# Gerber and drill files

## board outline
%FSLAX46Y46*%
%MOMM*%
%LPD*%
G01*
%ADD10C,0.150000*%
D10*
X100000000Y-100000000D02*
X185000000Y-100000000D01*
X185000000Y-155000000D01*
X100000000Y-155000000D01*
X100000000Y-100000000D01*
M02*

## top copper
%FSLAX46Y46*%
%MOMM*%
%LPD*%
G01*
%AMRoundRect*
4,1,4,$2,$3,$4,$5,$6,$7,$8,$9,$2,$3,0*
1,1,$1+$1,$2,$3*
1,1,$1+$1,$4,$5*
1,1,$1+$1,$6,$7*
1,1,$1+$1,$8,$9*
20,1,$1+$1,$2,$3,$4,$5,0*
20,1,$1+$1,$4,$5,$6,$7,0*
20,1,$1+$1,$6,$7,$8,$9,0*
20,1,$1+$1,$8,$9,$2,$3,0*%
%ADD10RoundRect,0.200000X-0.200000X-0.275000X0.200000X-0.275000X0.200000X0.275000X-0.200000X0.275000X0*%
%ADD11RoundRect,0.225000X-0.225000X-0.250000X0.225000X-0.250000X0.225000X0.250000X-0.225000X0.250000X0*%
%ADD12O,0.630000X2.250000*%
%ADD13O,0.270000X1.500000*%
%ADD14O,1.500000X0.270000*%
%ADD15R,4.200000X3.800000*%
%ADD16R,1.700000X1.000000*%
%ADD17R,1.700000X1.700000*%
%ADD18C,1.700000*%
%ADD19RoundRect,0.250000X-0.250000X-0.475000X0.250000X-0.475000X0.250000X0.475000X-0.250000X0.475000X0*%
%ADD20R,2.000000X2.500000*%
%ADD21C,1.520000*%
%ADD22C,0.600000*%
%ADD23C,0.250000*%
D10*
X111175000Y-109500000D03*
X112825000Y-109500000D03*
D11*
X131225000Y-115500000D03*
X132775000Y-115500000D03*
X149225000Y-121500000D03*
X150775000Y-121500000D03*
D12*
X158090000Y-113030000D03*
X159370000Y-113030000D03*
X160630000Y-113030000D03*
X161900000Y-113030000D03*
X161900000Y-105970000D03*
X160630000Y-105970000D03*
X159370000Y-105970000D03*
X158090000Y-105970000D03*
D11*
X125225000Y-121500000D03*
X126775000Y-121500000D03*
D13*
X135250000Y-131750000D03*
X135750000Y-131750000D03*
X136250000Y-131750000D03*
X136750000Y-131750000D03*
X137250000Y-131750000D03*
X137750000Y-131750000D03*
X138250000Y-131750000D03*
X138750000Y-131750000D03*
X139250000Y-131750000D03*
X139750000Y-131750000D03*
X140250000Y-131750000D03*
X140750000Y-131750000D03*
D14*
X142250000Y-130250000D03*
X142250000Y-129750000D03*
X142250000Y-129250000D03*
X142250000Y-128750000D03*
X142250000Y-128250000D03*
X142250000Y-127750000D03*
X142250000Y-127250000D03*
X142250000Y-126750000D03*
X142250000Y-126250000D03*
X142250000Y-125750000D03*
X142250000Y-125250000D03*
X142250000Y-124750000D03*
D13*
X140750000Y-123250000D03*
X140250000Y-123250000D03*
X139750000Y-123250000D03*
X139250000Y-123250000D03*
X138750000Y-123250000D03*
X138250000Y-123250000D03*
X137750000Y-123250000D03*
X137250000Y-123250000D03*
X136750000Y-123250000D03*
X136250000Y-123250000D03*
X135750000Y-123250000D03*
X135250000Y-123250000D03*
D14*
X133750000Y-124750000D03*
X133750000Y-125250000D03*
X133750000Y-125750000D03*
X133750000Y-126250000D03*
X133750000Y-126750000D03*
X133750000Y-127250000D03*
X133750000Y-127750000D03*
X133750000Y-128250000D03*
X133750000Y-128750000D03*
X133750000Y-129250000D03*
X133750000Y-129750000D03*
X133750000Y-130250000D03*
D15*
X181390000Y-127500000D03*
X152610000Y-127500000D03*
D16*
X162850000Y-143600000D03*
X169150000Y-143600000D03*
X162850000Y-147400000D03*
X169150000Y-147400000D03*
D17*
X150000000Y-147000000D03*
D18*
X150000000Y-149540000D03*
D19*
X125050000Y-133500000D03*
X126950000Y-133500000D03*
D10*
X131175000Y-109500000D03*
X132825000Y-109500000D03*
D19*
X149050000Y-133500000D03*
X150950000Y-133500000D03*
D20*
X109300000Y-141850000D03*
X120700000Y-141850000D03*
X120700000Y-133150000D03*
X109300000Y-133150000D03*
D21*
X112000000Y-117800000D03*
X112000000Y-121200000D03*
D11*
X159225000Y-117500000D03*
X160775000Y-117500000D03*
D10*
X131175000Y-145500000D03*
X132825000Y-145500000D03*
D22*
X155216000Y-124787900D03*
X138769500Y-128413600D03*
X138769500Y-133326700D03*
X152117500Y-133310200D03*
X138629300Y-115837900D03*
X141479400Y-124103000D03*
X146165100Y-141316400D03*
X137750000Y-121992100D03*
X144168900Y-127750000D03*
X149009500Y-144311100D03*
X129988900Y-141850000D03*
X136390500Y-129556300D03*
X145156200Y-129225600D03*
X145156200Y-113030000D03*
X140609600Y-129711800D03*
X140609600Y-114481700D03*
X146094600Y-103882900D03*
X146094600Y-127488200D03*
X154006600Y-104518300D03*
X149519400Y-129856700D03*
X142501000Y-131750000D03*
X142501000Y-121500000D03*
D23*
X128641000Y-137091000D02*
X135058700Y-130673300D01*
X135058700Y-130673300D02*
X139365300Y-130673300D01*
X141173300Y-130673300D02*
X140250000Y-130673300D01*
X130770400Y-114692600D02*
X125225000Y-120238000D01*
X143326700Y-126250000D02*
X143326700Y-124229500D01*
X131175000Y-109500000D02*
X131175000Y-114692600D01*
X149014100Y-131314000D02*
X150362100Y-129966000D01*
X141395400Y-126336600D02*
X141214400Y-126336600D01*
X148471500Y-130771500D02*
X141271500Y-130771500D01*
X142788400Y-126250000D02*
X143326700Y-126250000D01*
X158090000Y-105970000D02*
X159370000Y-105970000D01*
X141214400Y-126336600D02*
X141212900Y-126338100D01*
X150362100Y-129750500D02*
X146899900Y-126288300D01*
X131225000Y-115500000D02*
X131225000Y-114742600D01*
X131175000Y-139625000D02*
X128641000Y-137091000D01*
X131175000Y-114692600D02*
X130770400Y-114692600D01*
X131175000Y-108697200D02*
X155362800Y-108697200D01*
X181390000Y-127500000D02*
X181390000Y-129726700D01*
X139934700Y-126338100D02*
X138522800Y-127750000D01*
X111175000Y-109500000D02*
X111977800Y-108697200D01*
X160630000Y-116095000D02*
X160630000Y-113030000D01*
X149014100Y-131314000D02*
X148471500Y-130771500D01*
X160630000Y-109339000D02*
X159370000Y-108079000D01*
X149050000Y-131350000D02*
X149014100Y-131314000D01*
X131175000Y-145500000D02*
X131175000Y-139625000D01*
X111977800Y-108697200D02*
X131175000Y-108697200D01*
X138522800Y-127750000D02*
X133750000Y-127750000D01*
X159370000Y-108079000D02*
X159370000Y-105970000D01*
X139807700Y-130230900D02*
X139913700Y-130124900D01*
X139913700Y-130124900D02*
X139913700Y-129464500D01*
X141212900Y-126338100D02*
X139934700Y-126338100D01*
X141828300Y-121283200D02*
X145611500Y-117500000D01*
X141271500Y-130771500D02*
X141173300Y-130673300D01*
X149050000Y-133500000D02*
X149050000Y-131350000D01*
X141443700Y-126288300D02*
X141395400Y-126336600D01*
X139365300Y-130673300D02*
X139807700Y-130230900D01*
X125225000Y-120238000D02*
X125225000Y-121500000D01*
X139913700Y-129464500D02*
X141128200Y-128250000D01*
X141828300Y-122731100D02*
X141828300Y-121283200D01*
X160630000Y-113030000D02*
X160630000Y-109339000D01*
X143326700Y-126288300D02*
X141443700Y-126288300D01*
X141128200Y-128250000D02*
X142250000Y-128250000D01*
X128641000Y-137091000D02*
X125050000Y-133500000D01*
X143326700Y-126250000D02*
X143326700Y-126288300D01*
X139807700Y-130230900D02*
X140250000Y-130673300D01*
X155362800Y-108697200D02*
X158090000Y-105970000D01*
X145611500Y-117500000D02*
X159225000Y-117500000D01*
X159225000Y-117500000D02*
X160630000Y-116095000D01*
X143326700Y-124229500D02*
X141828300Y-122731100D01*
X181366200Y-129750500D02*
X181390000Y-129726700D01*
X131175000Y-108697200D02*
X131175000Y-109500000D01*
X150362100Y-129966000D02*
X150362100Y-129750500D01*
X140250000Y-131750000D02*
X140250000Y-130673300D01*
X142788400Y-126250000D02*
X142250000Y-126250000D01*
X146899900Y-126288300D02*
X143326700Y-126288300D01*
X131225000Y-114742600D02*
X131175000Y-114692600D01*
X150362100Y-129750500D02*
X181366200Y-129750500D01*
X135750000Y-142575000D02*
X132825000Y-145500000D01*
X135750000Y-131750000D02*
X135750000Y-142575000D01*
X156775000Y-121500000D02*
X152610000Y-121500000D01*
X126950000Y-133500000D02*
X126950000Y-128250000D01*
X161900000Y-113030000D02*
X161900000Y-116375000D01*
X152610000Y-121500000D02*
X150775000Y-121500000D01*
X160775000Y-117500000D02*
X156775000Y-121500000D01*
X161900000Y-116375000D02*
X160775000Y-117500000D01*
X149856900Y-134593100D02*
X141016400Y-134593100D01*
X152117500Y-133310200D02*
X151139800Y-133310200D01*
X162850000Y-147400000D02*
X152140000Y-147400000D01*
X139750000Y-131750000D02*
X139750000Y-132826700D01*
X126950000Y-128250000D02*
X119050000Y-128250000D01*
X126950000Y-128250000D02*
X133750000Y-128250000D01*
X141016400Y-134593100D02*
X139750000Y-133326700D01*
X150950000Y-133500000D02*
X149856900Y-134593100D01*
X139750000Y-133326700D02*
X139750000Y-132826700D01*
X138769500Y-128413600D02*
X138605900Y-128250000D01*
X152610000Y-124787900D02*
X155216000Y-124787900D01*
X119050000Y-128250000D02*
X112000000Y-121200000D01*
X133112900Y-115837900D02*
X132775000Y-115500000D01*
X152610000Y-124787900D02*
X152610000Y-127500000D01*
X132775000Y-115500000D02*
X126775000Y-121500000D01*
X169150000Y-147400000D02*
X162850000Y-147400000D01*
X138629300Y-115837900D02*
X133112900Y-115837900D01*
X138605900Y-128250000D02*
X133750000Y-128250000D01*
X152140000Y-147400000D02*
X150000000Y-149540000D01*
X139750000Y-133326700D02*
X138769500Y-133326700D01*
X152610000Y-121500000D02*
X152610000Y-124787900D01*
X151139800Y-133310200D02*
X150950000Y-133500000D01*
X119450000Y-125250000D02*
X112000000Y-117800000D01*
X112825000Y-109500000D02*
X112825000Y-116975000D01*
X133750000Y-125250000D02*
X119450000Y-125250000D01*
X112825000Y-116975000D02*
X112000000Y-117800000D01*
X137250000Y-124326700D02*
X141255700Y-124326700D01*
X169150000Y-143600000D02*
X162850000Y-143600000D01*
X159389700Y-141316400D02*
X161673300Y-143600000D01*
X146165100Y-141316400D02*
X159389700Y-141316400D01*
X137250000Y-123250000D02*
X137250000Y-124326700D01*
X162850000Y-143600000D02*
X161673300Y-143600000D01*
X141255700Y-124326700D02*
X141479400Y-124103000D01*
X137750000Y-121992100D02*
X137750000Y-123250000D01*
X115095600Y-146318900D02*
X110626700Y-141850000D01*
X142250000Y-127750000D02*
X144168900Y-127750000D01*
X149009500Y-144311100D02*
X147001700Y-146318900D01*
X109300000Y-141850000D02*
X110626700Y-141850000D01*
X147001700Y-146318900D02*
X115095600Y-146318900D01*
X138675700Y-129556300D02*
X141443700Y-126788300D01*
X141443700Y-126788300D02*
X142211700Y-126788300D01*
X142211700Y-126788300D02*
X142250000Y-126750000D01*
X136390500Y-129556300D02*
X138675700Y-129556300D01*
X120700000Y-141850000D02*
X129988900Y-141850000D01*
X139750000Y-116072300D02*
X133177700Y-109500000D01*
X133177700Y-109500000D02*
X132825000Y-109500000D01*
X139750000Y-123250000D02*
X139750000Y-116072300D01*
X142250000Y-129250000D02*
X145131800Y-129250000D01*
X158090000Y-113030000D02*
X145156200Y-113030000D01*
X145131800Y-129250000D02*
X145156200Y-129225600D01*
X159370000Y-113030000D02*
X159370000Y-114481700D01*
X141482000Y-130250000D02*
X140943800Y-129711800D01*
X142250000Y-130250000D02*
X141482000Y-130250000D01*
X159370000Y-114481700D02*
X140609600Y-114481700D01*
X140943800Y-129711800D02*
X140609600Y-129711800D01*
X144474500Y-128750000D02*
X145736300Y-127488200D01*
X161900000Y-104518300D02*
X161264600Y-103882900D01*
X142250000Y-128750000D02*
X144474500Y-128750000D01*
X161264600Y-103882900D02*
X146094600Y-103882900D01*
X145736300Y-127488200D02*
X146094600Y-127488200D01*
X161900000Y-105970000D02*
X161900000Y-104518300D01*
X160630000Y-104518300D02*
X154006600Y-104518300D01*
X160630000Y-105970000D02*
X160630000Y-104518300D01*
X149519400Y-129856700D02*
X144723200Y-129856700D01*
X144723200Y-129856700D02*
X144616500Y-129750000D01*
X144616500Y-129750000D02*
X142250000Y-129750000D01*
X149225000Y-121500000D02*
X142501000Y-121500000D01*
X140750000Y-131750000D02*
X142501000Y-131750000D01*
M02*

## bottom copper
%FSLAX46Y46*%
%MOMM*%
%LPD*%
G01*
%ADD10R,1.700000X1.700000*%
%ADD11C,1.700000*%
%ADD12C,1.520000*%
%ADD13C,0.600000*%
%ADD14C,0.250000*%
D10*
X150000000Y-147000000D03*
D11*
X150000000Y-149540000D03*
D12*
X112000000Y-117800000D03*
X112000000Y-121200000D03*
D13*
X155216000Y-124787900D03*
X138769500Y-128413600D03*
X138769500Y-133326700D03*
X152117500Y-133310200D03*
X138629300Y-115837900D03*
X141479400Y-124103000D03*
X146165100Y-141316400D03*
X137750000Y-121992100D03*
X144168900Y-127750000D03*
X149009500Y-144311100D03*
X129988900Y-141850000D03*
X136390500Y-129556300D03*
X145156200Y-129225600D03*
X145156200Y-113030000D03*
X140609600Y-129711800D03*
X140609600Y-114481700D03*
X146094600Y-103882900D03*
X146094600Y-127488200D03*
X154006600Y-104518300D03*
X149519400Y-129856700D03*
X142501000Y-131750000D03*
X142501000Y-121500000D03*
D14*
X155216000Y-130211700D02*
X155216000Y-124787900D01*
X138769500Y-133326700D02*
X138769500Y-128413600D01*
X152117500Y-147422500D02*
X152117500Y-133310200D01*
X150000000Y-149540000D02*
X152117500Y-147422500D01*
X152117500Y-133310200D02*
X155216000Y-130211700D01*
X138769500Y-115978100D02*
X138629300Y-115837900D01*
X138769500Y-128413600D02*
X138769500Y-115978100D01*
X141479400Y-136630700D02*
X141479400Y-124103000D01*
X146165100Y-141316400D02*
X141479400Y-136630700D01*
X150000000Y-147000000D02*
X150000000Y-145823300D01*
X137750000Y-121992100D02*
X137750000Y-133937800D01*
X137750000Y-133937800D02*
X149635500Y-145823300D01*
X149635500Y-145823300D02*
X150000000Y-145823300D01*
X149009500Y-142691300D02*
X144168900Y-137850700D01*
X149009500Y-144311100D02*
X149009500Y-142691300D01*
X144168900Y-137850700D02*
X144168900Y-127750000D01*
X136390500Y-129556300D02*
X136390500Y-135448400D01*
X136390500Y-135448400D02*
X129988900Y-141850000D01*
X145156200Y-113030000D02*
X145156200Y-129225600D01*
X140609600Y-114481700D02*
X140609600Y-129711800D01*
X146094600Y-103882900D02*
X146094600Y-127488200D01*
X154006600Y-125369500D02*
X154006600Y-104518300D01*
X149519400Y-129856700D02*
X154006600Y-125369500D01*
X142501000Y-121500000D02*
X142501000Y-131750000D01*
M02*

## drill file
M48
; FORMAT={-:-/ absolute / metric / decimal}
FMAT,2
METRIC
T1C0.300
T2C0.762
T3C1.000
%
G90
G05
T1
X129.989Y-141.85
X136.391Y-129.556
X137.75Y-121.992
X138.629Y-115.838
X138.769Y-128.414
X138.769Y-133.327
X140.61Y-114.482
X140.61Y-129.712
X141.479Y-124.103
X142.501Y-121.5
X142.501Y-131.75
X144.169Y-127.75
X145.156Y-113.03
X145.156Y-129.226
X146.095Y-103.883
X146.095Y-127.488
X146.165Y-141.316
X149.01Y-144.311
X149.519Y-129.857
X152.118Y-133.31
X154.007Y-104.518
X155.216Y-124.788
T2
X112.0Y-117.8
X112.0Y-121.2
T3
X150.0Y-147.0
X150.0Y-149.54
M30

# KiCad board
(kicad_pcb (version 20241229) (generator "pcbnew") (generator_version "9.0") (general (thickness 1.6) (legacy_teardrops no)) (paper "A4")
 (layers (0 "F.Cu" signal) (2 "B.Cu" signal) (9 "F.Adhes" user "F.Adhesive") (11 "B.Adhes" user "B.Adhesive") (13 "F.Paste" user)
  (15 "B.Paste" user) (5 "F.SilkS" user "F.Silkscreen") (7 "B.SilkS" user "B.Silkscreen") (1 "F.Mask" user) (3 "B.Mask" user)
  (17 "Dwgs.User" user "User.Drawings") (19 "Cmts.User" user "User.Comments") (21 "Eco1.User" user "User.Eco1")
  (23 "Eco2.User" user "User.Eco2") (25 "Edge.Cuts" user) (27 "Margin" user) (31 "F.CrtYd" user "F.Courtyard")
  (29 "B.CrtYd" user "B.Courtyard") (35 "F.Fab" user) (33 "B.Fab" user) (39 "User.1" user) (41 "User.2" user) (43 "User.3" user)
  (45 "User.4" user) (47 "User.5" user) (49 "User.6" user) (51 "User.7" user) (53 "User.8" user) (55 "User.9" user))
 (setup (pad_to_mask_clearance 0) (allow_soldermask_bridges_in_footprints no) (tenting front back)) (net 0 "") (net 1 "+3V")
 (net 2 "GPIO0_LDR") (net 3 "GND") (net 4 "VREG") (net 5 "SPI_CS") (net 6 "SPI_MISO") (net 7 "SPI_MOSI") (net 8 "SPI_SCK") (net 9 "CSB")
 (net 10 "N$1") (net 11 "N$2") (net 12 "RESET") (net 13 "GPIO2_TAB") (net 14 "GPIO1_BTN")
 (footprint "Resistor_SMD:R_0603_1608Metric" (layer "F.Cu") (at 112 109.5)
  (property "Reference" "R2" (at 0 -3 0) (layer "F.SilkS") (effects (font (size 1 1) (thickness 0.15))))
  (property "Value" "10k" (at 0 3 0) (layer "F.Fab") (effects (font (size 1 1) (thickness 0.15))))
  (pad "1" smd roundrect (at -0.825 0) (size 0.8 0.95) (layers "F.Cu" "F.Mask" "F.Paste") (roundrect_rratio 0.25) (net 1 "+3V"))
  (pad "2" smd roundrect (at 0.825 0) (size 0.8 0.95) (layers "F.Cu" "F.Mask" "F.Paste") (roundrect_rratio 0.25) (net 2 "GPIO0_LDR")))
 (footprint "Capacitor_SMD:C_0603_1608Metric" (layer "F.Cu") (at 132 115.5)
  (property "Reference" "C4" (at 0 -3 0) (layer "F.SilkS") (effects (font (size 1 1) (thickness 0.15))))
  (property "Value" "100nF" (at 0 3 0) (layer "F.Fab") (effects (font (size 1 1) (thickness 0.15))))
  (pad "1" smd roundrect (at -0.775 0) (size 0.9 0.95) (layers "F.Cu" "F.Mask" "F.Paste") (roundrect_rratio 0.25) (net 1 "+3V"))
  (pad "2" smd roundrect (at 0.775 0) (size 0.9 0.95) (layers "F.Cu" "F.Mask" "F.Paste") (roundrect_rratio 0.25) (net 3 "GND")))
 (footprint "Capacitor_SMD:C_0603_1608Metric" (layer "F.Cu") (at 150 121.5)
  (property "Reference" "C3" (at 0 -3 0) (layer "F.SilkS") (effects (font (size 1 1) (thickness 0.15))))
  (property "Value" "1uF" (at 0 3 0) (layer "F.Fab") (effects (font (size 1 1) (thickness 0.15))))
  (pad "1" smd roundrect (at -0.775 0) (size 0.9 0.95) (layers "F.Cu" "F.Mask" "F.Paste") (roundrect_rratio 0.25) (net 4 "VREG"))
  (pad "2" smd roundrect (at 0.775 0) (size 0.9 0.95) (layers "F.Cu" "F.Mask" "F.Paste") (roundrect_rratio 0.25) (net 3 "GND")))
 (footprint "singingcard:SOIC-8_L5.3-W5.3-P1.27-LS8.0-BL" (layer "F.Cu") (at 160 109.5)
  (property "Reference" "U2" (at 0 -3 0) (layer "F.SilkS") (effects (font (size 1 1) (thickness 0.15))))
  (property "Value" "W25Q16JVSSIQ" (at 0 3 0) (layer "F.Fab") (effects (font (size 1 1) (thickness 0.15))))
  (pad "1" smd oval (at -1.91 3.53) (size 0.63 2.25) (layers "F.Cu" "F.Mask" "F.Paste") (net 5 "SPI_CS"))
  (pad "2" smd oval (at -0.63 3.53) (size 0.63 2.25) (layers "F.Cu" "F.Mask" "F.Paste") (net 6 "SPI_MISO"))
  (pad "3" smd oval (at 0.63 3.53) (size 0.63 2.25) (layers "F.Cu" "F.Mask" "F.Paste") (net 1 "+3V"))
  (pad "4" smd oval (at 1.9 3.53) (size 0.63 2.25) (layers "F.Cu" "F.Mask" "F.Paste") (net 3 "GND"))
  (pad "5" smd oval (at 1.9 -3.53) (size 0.63 2.25) (layers "F.Cu" "F.Mask" "F.Paste") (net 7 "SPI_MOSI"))
  (pad "6" smd oval (at 0.63 -3.53) (size 0.63 2.25) (layers "F.Cu" "F.Mask" "F.Paste") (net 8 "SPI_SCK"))
  (pad "7" smd oval (at -0.63 -3.53) (size 0.63 2.25) (layers "F.Cu" "F.Mask" "F.Paste") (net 1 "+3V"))
  (pad "8" smd oval (at -1.91 -3.53) (size 0.63 2.25) (layers "F.Cu" "F.Mask" "F.Paste") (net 1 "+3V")))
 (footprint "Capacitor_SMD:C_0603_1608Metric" (layer "F.Cu") (at 126 121.5)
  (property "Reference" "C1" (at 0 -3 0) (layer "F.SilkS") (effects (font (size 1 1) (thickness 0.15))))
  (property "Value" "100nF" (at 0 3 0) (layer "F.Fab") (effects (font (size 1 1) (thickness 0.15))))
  (pad "1" smd roundrect (at -0.775 0) (size 0.9 0.95) (layers "F.Cu" "F.Mask" "F.Paste") (roundrect_rratio 0.25) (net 1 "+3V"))
  (pad "2" smd roundrect (at 0.775 0) (size 0.9 0.95) (layers "F.Cu" "F.Mask" "F.Paste") (roundrect_rratio 0.25) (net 3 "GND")))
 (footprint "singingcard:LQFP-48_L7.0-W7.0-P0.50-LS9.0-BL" (layer "F.Cu") (at 138 127.5)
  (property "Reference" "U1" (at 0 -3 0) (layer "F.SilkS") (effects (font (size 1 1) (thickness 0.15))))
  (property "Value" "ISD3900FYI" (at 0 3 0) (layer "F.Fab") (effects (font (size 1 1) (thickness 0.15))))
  (pad "1" smd oval (at -2.75 4.25) (size 0.27 1.5) (layers "F.Cu" "F.Mask" "F.Paste"))
  (pad "2" smd oval (at -2.25 4.25) (size 0.27 1.5) (layers "F.Cu" "F.Mask" "F.Paste") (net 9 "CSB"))
  (pad "3" smd oval (at -1.75 4.25) (size 0.27 1.5) (layers "F.Cu" "F.Mask" "F.Paste"))
  (pad "4" smd oval (at -1.25 4.25) (size 0.27 1.5) (layers "F.Cu" "F.Mask" "F.Paste"))
  (pad "5" smd oval (at -0.75 4.25) (size 0.27 1.5) (layers "F.Cu" "F.Mask" "F.Paste"))
  (pad "6" smd oval (at -0.25 4.25) (size 0.27 1.5) (layers "F.Cu" "F.Mask" "F.Paste"))
  (pad "7" smd oval (at 0.25 4.25) (size 0.27 1.5) (layers "F.Cu" "F.Mask" "F.Paste"))
  (pad "8" smd oval (at 0.75 4.25) (size 0.27 1.5) (layers "F.Cu" "F.Mask" "F.Paste"))
  (pad "9" smd oval (at 1.25 4.25) (size 0.27 1.5) (layers "F.Cu" "F.Mask" "F.Paste"))
  (pad "10" smd oval (at 1.75 4.25) (size 0.27 1.5) (layers "F.Cu" "F.Mask" "F.Paste") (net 3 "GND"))
  (pad "11" smd oval (at 2.25 4.25) (size 0.27 1.5) (layers "F.Cu" "F.Mask" "F.Paste") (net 1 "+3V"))
  (pad "12" smd oval (at 2.75 4.25) (size 0.27 1.5) (layers "F.Cu" "F.Mask" "F.Paste") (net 4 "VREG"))
  (pad "13" smd oval (at 4.25 2.75) (size 1.5 0.27) (layers "F.Cu" "F.Mask" "F.Paste") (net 6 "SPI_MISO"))
  (pad "14" smd oval (at 4.25 2.25) (size 1.5 0.27) (layers "F.Cu" "F.Mask" "F.Paste") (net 8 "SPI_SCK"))
  (pad "15" smd oval (at 4.25 1.75) (size 1.5 0.27) (layers "F.Cu" "F.Mask" "F.Paste") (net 5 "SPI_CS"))
  (pad "16" smd oval (at 4.25 1.25) (size 1.5 0.27) (layers "F.Cu" "F.Mask" "F.Paste") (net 7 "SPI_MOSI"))
  (pad "17" smd oval (at 4.25 0.75) (size 1.5 0.27) (layers "F.Cu" "F.Mask" "F.Paste") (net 1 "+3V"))
  (pad "18" smd oval (at 4.25 0.25) (size 1.5 0.27) (layers "F.Cu" "F.Mask" "F.Paste") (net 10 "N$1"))
  (pad "19" smd oval (at 4.25 -0.25) (size 1.5 0.27) (layers "F.Cu" "F.Mask" "F.Paste"))
  (pad "20" smd oval (at 4.25 -0.75) (size 1.5 0.27) (layers "F.Cu" "F.Mask" "F.Paste") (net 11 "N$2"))
  (pad "21" smd oval (at 4.25 -1.25) (size 1.5 0.27) (layers "F.Cu" "F.Mask" "F.Paste") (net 1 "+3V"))
  (pad "22" smd oval (at 4.25 -1.75) (size 1.5 0.27) (layers "F.Cu" "F.Mask" "F.Paste"))
  (pad "23" smd oval (at 4.25 -2.25) (size 1.5 0.27) (layers "F.Cu" "F.Mask" "F.Paste"))
  (pad "24" smd oval (at 4.25 -2.75) (size 1.5 0.27) (layers "F.Cu" "F.Mask" "F.Paste"))
  (pad "25" smd oval (at 2.75 -4.25) (size 0.27 1.5) (layers "F.Cu" "F.Mask" "F.Paste"))
  (pad "26" smd oval (at 2.25 -4.25) (size 0.27 1.5) (layers "F.Cu" "F.Mask" "F.Paste"))
  (pad "27" smd oval (at 1.75 -4.25) (size 0.27 1.5) (layers "F.Cu" "F.Mask" "F.Paste") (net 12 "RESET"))
  (pad "28" smd oval (at 1.25 -4.25) (size 0.27 1.5) (layers "F.Cu" "F.Mask" "F.Paste"))
  (pad "29" smd oval (at 0.75 -4.25) (size 0.27 1.5) (layers "F.Cu" "F.Mask" "F.Paste"))
  (pad "30" smd oval (at 0.25 -4.25) (size 0.27 1.5) (layers "F.Cu" "F.Mask" "F.Paste"))
  (pad "31" smd oval (at -0.25 -4.25) (size 0.27 1.5) (layers "F.Cu" "F.Mask" "F.Paste") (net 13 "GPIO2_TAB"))
  (pad "32" smd oval (at -0.75 -4.25) (size 0.27 1.5) (layers "F.Cu" "F.Mask" "F.Paste") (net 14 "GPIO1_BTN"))
  (pad "33" smd oval (at -1.25 -4.25) (size 0.27 1.5) (layers "F.Cu" "F.Mask" "F.Paste"))
  (pad "34" smd oval (at -1.75 -4.25) (size 0.27 1.5) (layers "F.Cu" "F.Mask" "F.Paste"))
  (pad "35" smd oval (at -2.25 -4.25) (size 0.27 1.5) (layers "F.Cu" "F.Mask" "F.Paste"))
  (pad "36" smd oval (at -2.75 -4.25) (size 0.27 1.5) (layers "F.Cu" "F.Mask" "F.Paste"))
  (pad "37" smd oval (at -4.25 -2.75) (size 1.5 0.27) (layers "F.Cu" "F.Mask" "F.Paste"))
  (pad "38" smd oval (at -4.25 -2.25) (size 1.5 0.27) (layers "F.Cu" "F.Mask" "F.Paste") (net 2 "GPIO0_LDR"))
  (pad "39" smd oval (at -4.25 -1.75) (size 1.5 0.27) (layers "F.Cu" "F.Mask" "F.Paste"))
  (pad "40" smd oval (at -4.25 -1.25) (size 1.5 0.27) (layers "F.Cu" "F.Mask" "F.Paste"))
  (pad "41" smd oval (at -4.25 -0.75) (size 1.5 0.27) (layers "F.Cu" "F.Mask" "F.Paste"))
  (pad "42" smd oval (at -4.25 -0.25) (size 1.5 0.27) (layers "F.Cu" "F.Mask" "F.Paste"))
  (pad "43" smd oval (at -4.25 0.25) (size 1.5 0.27) (layers "F.Cu" "F.Mask" "F.Paste") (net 1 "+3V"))
  (pad "44" smd oval (at -4.25 0.75) (size 1.5 0.27) (layers "F.Cu" "F.Mask" "F.Paste") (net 3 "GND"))
  (pad "45" smd oval (at -4.25 1.25) (size 1.5 0.27) (layers "F.Cu" "F.Mask" "F.Paste"))
  (pad "46" smd oval (at -4.25 1.75) (size 1.5 0.27) (layers "F.Cu" "F.Mask" "F.Paste"))
  (pad "47" smd oval (at -4.25 2.25) (size 1.5 0.27) (layers "F.Cu" "F.Mask" "F.Paste"))
  (pad "48" smd oval (at -4.25 2.75) (size 1.5 0.27) (layers "F.Cu" "F.Mask" "F.Paste")))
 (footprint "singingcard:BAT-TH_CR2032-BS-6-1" (layer "F.Cu") (at 167 127.5)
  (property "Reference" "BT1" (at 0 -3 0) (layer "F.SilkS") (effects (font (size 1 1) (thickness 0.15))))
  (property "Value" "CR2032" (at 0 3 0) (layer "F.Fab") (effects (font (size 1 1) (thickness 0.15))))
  (pad "1" smd rect (at 14.39 0) (size 4.2 3.8) (layers "F.Cu" "F.Mask" "F.Paste") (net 1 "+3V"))
  (pad "2" smd rect (at -14.39 0) (size 4.2 3.8) (layers "F.Cu" "F.Mask" "F.Paste") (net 3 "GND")))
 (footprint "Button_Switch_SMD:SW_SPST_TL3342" (layer "F.Cu") (at 166 145.5)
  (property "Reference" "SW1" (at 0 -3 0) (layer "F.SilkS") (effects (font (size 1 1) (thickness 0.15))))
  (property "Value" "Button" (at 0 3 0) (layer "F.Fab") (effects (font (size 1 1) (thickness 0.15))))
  (pad "1" smd rect (at -3.15 -1.9) (size 1.7 1) (layers "F.Cu" "F.Mask" "F.Paste") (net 14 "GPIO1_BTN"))
  (pad "1" smd rect (at 3.15 -1.9) (size 1.7 1) (layers "F.Cu" "F.Mask" "F.Paste") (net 14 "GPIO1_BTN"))
  (pad "2" smd rect (at -3.15 1.9) (size 1.7 1) (layers "F.Cu" "F.Mask" "F.Paste") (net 3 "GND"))
  (pad "2" smd rect (at 3.15 1.9) (size 1.7 1) (layers "F.Cu" "F.Mask" "F.Paste") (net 3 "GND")))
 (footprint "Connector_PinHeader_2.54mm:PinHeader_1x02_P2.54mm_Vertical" (layer "F.Cu") (at 150 147)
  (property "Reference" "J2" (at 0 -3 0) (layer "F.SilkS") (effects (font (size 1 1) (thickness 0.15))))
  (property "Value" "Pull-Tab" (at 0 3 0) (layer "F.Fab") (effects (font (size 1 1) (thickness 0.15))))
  (pad "1" thru_hole rect (at 0 0) (size 1.7 1.7) (drill 1) (layers "*.Cu" "*.Mask") (remove_unused_layers no) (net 13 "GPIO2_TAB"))
  (pad "2" thru_hole circle (at 0 2.54) (size 1.7 1.7) (drill 1) (layers "*.Cu" "*.Mask") (remove_unused_layers no) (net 3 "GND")))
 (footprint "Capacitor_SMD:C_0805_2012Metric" (layer "F.Cu") (at 126 133.5)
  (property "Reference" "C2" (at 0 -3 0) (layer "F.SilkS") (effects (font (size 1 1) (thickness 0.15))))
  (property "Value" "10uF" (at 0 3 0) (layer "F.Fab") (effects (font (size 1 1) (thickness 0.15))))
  (pad "1" smd roundrect (at -0.95 0) (size 1 1.45) (layers "F.Cu" "F.Mask" "F.Paste") (roundrect_rratio 0.25) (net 1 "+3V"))
  (pad "2" smd roundrect (at 0.95 0) (size 1 1.45) (layers "F.Cu" "F.Mask" "F.Paste") (roundrect_rratio 0.25) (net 3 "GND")))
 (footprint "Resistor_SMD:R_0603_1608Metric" (layer "F.Cu") (at 132 109.5)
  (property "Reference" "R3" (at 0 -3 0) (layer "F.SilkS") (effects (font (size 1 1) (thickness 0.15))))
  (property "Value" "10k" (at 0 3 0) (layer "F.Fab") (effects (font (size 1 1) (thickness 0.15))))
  (pad "1" smd roundrect (at -0.825 0) (size 0.8 0.95) (layers "F.Cu" "F.Mask" "F.Paste") (roundrect_rratio 0.25) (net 1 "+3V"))
  (pad "2" smd roundrect (at 0.825 0) (size 0.8 0.95) (layers "F.Cu" "F.Mask" "F.Paste") (roundrect_rratio 0.25) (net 12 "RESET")))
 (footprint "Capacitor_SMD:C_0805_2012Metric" (layer "F.Cu") (at 150 133.5)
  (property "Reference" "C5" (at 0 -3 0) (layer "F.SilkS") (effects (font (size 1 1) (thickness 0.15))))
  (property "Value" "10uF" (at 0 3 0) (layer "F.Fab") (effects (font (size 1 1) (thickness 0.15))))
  (pad "1" smd roundrect (at -0.95 0) (size 1 1.45) (layers "F.Cu" "F.Mask" "F.Paste") (roundrect_rratio 0.25) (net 1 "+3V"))
  (pad "2" smd roundrect (at 0.95 0) (size 1 1.45) (layers "F.Cu" "F.Mask" "F.Paste") (roundrect_rratio 0.25) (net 3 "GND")))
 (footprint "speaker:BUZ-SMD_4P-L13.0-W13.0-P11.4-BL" (layer "F.Cu") (at 115 137.5)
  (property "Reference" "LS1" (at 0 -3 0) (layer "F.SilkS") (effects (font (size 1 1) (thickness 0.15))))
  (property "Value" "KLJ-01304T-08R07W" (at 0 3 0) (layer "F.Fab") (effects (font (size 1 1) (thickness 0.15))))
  (pad "1" smd rect (at -5.7 4.35) (size 2 2.5) (layers "F.Cu" "F.Mask" "F.Paste") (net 10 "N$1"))
  (pad "2" smd rect (at 5.7 4.35) (size 2 2.5) (layers "F.Cu" "F.Mask" "F.Paste") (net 11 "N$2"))
  (pad "3" smd rect (at 5.7 -4.35) (size 2 2.5) (layers "F.Cu" "F.Mask" "F.Paste"))
  (pad "4" smd rect (at -5.7 -4.35) (size 2 2.5) (layers "F.Cu" "F.Mask" "F.Paste")))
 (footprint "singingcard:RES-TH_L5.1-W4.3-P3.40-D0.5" (layer "F.Cu") (at 112 119.5)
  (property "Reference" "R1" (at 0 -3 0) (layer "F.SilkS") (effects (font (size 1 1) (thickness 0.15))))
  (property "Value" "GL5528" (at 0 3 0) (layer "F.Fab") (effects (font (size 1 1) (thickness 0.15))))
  (pad "1" thru_hole circle (at 0 -1.7 270) (size 1.52 1.52) (drill 0.762) (layers "*.Cu" "*.Mask") (remove_unused_layers no)
   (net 2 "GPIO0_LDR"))
  (pad "2" thru_hole circle (at 0 1.7 270) (size 1.52 1.52) (drill 0.762) (layers "*.Cu" "*.Mask") (remove_unused_layers no) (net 3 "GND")))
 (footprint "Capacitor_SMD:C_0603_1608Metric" (layer "F.Cu") (at 160 117.5)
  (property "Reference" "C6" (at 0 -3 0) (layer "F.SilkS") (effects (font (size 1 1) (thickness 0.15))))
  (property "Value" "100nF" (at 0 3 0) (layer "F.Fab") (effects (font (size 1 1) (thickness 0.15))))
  (pad "1" smd roundrect (at -0.775 0) (size 0.9 0.95) (layers "F.Cu" "F.Mask" "F.Paste") (roundrect_rratio 0.25) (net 1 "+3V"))
  (pad "2" smd roundrect (at 0.775 0) (size 0.9 0.95) (layers "F.Cu" "F.Mask" "F.Paste") (roundrect_rratio 0.25) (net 3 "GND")))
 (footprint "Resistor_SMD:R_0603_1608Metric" (layer "F.Cu") (at 132 145.5)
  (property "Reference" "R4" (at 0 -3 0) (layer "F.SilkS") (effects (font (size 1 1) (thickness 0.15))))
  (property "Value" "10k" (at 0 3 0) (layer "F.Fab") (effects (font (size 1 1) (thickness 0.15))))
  (pad "1" smd roundrect (at -0.825 0) (size 0.8 0.95) (layers "F.Cu" "F.Mask" "F.Paste") (roundrect_rratio 0.25) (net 1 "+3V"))
  (pad "2" smd roundrect (at 0.825 0) (size 0.8 0.95) (layers "F.Cu" "F.Mask" "F.Paste") (roundrect_rratio 0.25) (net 9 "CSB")))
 (gr_rect (start 100 100) (end 185 155) (stroke (width 0.15) (type default)) (fill no) (layer "Edge.Cuts"))
 (segment (start 128.641 137.091) (end 135.0587 130.6733) (width 0.25) (layer "F.Cu") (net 1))
 (segment (start 135.0587 130.6733) (end 139.3653 130.6733) (width 0.25) (layer "F.Cu") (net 1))
 (segment (start 141.1733 130.6733) (end 140.25 130.6733) (width 0.25) (layer "F.Cu") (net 1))
 (segment (start 130.7704 114.6926) (end 125.225 120.238) (width 0.25) (layer "F.Cu") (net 1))
 (segment (start 143.3267 126.25) (end 143.3267 124.2295) (width 0.25) (layer "F.Cu") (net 1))
 (segment (start 131.175 109.5) (end 131.175 114.6926) (width 0.25) (layer "F.Cu") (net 1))
 (segment (start 149.0141 131.314) (end 150.3621 129.966) (width 0.25) (layer "F.Cu") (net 1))
 (segment (start 141.3954 126.3366) (end 141.2144 126.3366) (width 0.25) (layer "F.Cu") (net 1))
 (segment (start 148.4715 130.7715) (end 141.2715 130.7715) (width 0.25) (layer "F.Cu") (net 1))
 (segment (start 142.7884 126.25) (end 143.3267 126.25) (width 0.25) (layer "F.Cu") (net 1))
 (segment (start 158.09 105.97) (end 159.37 105.97) (width 0.25) (layer "F.Cu") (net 1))
 (segment (start 141.2144 126.3366) (end 141.2129 126.3381) (width 0.25) (layer "F.Cu") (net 1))
 (segment (start 150.3621 129.7505) (end 146.8999 126.2883) (width 0.25) (layer "F.Cu") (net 1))
 (segment (start 131.225 115.5) (end 131.225 114.7426) (width 0.25) (layer "F.Cu") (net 1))
 (segment (start 131.175 139.625) (end 128.641 137.091) (width 0.25) (layer "F.Cu") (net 1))
 (segment (start 131.175 114.6926) (end 130.7704 114.6926) (width 0.25) (layer "F.Cu") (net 1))
 (segment (start 131.175 108.6972) (end 155.3628 108.6972) (width 0.25) (layer "F.Cu") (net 1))
 (segment (start 181.39 127.5) (end 181.39 129.7267) (width 0.25) (layer "F.Cu") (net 1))
 (segment (start 139.9347 126.3381) (end 138.5228 127.75) (width 0.25) (layer "F.Cu") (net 1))
 (segment (start 111.175 109.5) (end 111.9778 108.6972) (width 0.25) (layer "F.Cu") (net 1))
 (segment (start 160.63 116.095) (end 160.63 113.03) (width 0.25) (layer "F.Cu") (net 1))
 (segment (start 149.0141 131.314) (end 148.4715 130.7715) (width 0.25) (layer "F.Cu") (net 1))
 (segment (start 160.63 109.339) (end 159.37 108.079) (width 0.25) (layer "F.Cu") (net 1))
 (segment (start 149.05 131.35) (end 149.0141 131.314) (width 0.25) (layer "F.Cu") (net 1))
 (segment (start 131.175 145.5) (end 131.175 139.625) (width 0.25) (layer "F.Cu") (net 1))
 (segment (start 111.9778 108.6972) (end 131.175 108.6972) (width 0.25) (layer "F.Cu") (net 1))
 (segment (start 138.5228 127.75) (end 133.75 127.75) (width 0.25) (layer "F.Cu") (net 1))
 (segment (start 159.37 108.079) (end 159.37 105.97) (width 0.25) (layer "F.Cu") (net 1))
 (segment (start 139.8077 130.2309) (end 139.9137 130.1249) (width 0.25) (layer "F.Cu") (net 1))
 (segment (start 139.9137 130.1249) (end 139.9137 129.4645) (width 0.25) (layer "F.Cu") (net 1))
 (segment (start 141.2129 126.3381) (end 139.9347 126.3381) (width 0.25) (layer "F.Cu") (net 1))
 (segment (start 141.8283 121.2832) (end 145.6115 117.5) (width 0.25) (layer "F.Cu") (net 1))
 (segment (start 141.2715 130.7715) (end 141.1733 130.6733) (width 0.25) (layer "F.Cu") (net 1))
 (segment (start 149.05 133.5) (end 149.05 131.35) (width 0.25) (layer "F.Cu") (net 1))
 (segment (start 141.4437 126.2883) (end 141.3954 126.3366) (width 0.25) (layer "F.Cu") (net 1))
 (segment (start 139.3653 130.6733) (end 139.8077 130.2309) (width 0.25) (layer "F.Cu") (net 1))
 (segment (start 125.225 120.238) (end 125.225 121.5) (width 0.25) (layer "F.Cu") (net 1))
 (segment (start 139.9137 129.4645) (end 141.1282 128.25) (width 0.25) (layer "F.Cu") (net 1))
 (segment (start 141.8283 122.7311) (end 141.8283 121.2832) (width 0.25) (layer "F.Cu") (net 1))
 (segment (start 160.63 113.03) (end 160.63 109.339) (width 0.25) (layer "F.Cu") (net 1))
 (segment (start 143.3267 126.2883) (end 141.4437 126.2883) (width 0.25) (layer "F.Cu") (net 1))
 (segment (start 141.1282 128.25) (end 142.25 128.25) (width 0.25) (layer "F.Cu") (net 1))
 (segment (start 128.641 137.091) (end 125.05 133.5) (width 0.25) (layer "F.Cu") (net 1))
 (segment (start 143.3267 126.25) (end 143.3267 126.2883) (width 0.25) (layer "F.Cu") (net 1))
 (segment (start 139.8077 130.2309) (end 140.25 130.6733) (width 0.25) (layer "F.Cu") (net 1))
 (segment (start 155.3628 108.6972) (end 158.09 105.97) (width 0.25) (layer "F.Cu") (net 1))
 (segment (start 145.6115 117.5) (end 159.225 117.5) (width 0.25) (layer "F.Cu") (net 1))
 (segment (start 159.225 117.5) (end 160.63 116.095) (width 0.25) (layer "F.Cu") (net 1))
 (segment (start 143.3267 124.2295) (end 141.8283 122.7311) (width 0.25) (layer "F.Cu") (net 1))
 (segment (start 181.3662 129.7505) (end 181.39 129.7267) (width 0.25) (layer "F.Cu") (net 1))
 (segment (start 131.175 108.6972) (end 131.175 109.5) (width 0.25) (layer "F.Cu") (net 1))
 (segment (start 150.3621 129.966) (end 150.3621 129.7505) (width 0.25) (layer "F.Cu") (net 1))
 (segment (start 140.25 131.75) (end 140.25 130.6733) (width 0.25) (layer "F.Cu") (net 1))
 (segment (start 142.7884 126.25) (end 142.25 126.25) (width 0.25) (layer "F.Cu") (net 1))
 (segment (start 146.8999 126.2883) (end 143.3267 126.2883) (width 0.25) (layer "F.Cu") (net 1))
 (segment (start 131.225 114.7426) (end 131.175 114.6926) (width 0.25) (layer "F.Cu") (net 1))
 (segment (start 150.3621 129.7505) (end 181.3662 129.7505) (width 0.25) (layer "F.Cu") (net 1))
 (segment (start 135.75 142.575) (end 132.825 145.5) (width 0.25) (layer "F.Cu") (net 9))
 (segment (start 135.75 131.75) (end 135.75 142.575) (width 0.25) (layer "F.Cu") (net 9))
 (segment (start 156.775 121.5) (end 152.61 121.5) (width 0.25) (layer "F.Cu") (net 3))
 (segment (start 126.95 133.5) (end 126.95 128.25) (width 0.25) (layer "F.Cu") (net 3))
 (segment (start 161.9 113.03) (end 161.9 116.375) (width 0.25) (layer "F.Cu") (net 3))
 (segment (start 152.61 121.5) (end 150.775 121.5) (width 0.25) (layer "F.Cu") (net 3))
 (segment (start 160.775 117.5) (end 156.775 121.5) (width 0.25) (layer "F.Cu") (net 3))
 (segment (start 161.9 116.375) (end 160.775 117.5) (width 0.25) (layer "F.Cu") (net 3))
 (segment (start 149.8569 134.5931) (end 141.0164 134.5931) (width 0.25) (layer "F.Cu") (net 3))
 (segment (start 152.1175 133.3102) (end 151.1398 133.3102) (width 0.25) (layer "F.Cu") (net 3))
 (segment (start 162.85 147.4) (end 152.14 147.4) (width 0.25) (layer "F.Cu") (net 3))
 (segment (start 139.75 131.75) (end 139.75 132.8267) (width 0.25) (layer "F.Cu") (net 3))
 (segment (start 126.95 128.25) (end 119.05 128.25) (width 0.25) (layer "F.Cu") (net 3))
 (segment (start 126.95 128.25) (end 133.75 128.25) (width 0.25) (layer "F.Cu") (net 3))
 (segment (start 141.0164 134.5931) (end 139.75 133.3267) (width 0.25) (layer "F.Cu") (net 3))
 (segment (start 150.95 133.5) (end 149.8569 134.5931) (width 0.25) (layer "F.Cu") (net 3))
 (segment (start 139.75 133.3267) (end 139.75 132.8267) (width 0.25) (layer "F.Cu") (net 3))
 (segment (start 138.7695 128.4136) (end 138.6059 128.25) (width 0.25) (layer "F.Cu") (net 3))
 (segment (start 152.61 124.7879) (end 155.216 124.7879) (width 0.25) (layer "F.Cu") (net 3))
 (segment (start 119.05 128.25) (end 112 121.2) (width 0.25) (layer "F.Cu") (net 3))
 (segment (start 133.1129 115.8379) (end 132.775 115.5) (width 0.25) (layer "F.Cu") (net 3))
 (segment (start 152.61 124.7879) (end 152.61 127.5) (width 0.25) (layer "F.Cu") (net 3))
 (segment (start 132.775 115.5) (end 126.775 121.5) (width 0.25) (layer "F.Cu") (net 3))
 (segment (start 169.15 147.4) (end 162.85 147.4) (width 0.25) (layer "F.Cu") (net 3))
 (segment (start 138.6293 115.8379) (end 133.1129 115.8379) (width 0.25) (layer "F.Cu") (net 3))
 (segment (start 138.6059 128.25) (end 133.75 128.25) (width 0.25) (layer "F.Cu") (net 3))
 (segment (start 152.14 147.4) (end 150 149.54) (width 0.25) (layer "F.Cu") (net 3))
 (segment (start 139.75 133.3267) (end 138.7695 133.3267) (width 0.25) (layer "F.Cu") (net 3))
 (segment (start 152.61 121.5) (end 152.61 124.7879) (width 0.25) (layer "F.Cu") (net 3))
 (segment (start 151.1398 133.3102) (end 150.95 133.5) (width 0.25) (layer "F.Cu") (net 3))
 (via (at 155.216 124.7879) (size 0.6) (drill 0.3) (layers "F.Cu" "B.Cu") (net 3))
 (via (at 138.7695 128.4136) (size 0.6) (drill 0.3) (layers "F.Cu" "B.Cu") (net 3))
 (via (at 138.7695 133.3267) (size 0.6) (drill 0.3) (layers "F.Cu" "B.Cu") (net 3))
 (via (at 152.1175 133.3102) (size 0.6) (drill 0.3) (layers "F.Cu" "B.Cu") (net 3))
 (via (at 138.6293 115.8379) (size 0.6) (drill 0.3) (layers "F.Cu" "B.Cu") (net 3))
 (segment (start 155.216 130.2117) (end 155.216 124.7879) (width 0.25) (layer "B.Cu") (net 3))
 (segment (start 138.7695 133.3267) (end 138.7695 128.4136) (width 0.25) (layer "B.Cu") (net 3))
 (segment (start 152.1175 147.4225) (end 152.1175 133.3102) (width 0.25) (layer "B.Cu") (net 3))
 (segment (start 150 149.54) (end 152.1175 147.4225) (width 0.25) (layer "B.Cu") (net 3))
 (segment (start 152.1175 133.3102) (end 155.216 130.2117) (width 0.25) (layer "B.Cu") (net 3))
 (segment (start 138.7695 115.9781) (end 138.6293 115.8379) (width 0.25) (layer "B.Cu") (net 3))
 (segment (start 138.7695 128.4136) (end 138.7695 115.9781) (width 0.25) (layer "B.Cu") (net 3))
 (segment (start 119.45 125.25) (end 112 117.8) (width 0.25) (layer "F.Cu") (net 2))
 (segment (start 112.825 109.5) (end 112.825 116.975) (width 0.25) (layer "F.Cu") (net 2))
 (segment (start 133.75 125.25) (end 119.45 125.25) (width 0.25) (layer "F.Cu") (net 2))
 (segment (start 112.825 116.975) (end 112 117.8) (width 0.25) (layer "F.Cu") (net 2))
 (segment (start 137.25 124.3267) (end 141.2557 124.3267) (width 0.25) (layer "F.Cu") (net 14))
 (segment (start 169.15 143.6) (end 162.85 143.6) (width 0.25) (layer "F.Cu") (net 14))
 (segment (start 159.3897 141.3164) (end 161.6733 143.6) (width 0.25) (layer "F.Cu") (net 14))
 (segment (start 146.1651 141.3164) (end 159.3897 141.3164) (width 0.25) (layer "F.Cu") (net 14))
 (segment (start 137.25 123.25) (end 137.25 124.3267) (width 0.25) (layer "F.Cu") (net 14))
 (segment (start 162.85 143.6) (end 161.6733 143.6) (width 0.25) (layer "F.Cu") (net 14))
 (segment (start 141.2557 124.3267) (end 141.4794 124.103) (width 0.25) (layer "F.Cu") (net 14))
 (via (at 141.4794 124.103) (size 0.6) (drill 0.3) (layers "F.Cu" "B.Cu") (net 14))
 (via (at 146.1651 141.3164) (size 0.6) (drill 0.3) (layers "F.Cu" "B.Cu") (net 14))
 (segment (start 141.4794 136.6307) (end 141.4794 124.103) (width 0.25) (layer "B.Cu") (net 14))
 (segment (start 146.1651 141.3164) (end 141.4794 136.6307) (width 0.25) (layer "B.Cu") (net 14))
 (segment (start 137.75 121.9921) (end 137.75 123.25) (width 0.25) (layer "F.Cu") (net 13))
 (via (at 137.75 121.9921) (size 0.6) (drill 0.3) (layers "F.Cu" "B.Cu") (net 13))
 (segment (start 150 147) (end 150 145.8233) (width 0.25) (layer "B.Cu") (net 13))
 (segment (start 137.75 121.9921) (end 137.75 133.9378) (width 0.25) (layer "B.Cu") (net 13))
 (segment (start 137.75 133.9378) (end 149.6355 145.8233) (width 0.25) (layer "B.Cu") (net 13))
 (segment (start 149.6355 145.8233) (end 150 145.8233) (width 0.25) (layer "B.Cu") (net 13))
 (segment (start 115.0956 146.3189) (end 110.6267 141.85) (width 0.25) (layer "F.Cu") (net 10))
 (segment (start 142.25 127.75) (end 144.1689 127.75) (width 0.25) (layer "F.Cu") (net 10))
 (segment (start 149.0095 144.3111) (end 147.0017 146.3189) (width 0.25) (layer "F.Cu") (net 10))
 (segment (start 109.3 141.85) (end 110.6267 141.85) (width 0.25) (layer "F.Cu") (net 10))
 (segment (start 147.0017 146.3189) (end 115.0956 146.3189) (width 0.25) (layer "F.Cu") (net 10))
 (via (at 144.1689 127.75) (size 0.6) (drill 0.3) (layers "F.Cu" "B.Cu") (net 10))
 (via (at 149.0095 144.3111) (size 0.6) (drill 0.3) (layers "F.Cu" "B.Cu") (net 10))
 (segment (start 149.0095 142.6913) (end 144.1689 137.8507) (width 0.25) (layer "B.Cu") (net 10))
 (segment (start 149.0095 144.3111) (end 149.0095 142.6913) (width 0.25) (layer "B.Cu") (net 10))
 (segment (start 144.1689 137.8507) (end 144.1689 127.75) (width 0.25) (layer "B.Cu") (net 10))
 (segment (start 138.6757 129.5563) (end 141.4437 126.7883) (width 0.25) (layer "F.Cu") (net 11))
 (segment (start 141.4437 126.7883) (end 142.2117 126.7883) (width 0.25) (layer "F.Cu") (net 11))
 (segment (start 142.2117 126.7883) (end 142.25 126.75) (width 0.25) (layer "F.Cu") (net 11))
 (segment (start 136.3905 129.5563) (end 138.6757 129.5563) (width 0.25) (layer "F.Cu") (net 11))
 (segment (start 120.7 141.85) (end 129.9889 141.85) (width 0.25) (layer "F.Cu") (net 11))
 (via (at 129.9889 141.85) (size 0.6) (drill 0.3) (layers "F.Cu" "B.Cu") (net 11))
 (via (at 136.3905 129.5563) (size 0.6) (drill 0.3) (layers "F.Cu" "B.Cu") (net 11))
 (segment (start 136.3905 129.5563) (end 136.3905 135.4484) (width 0.25) (layer "B.Cu") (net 11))
 (segment (start 136.3905 135.4484) (end 129.9889 141.85) (width 0.25) (layer "B.Cu") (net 11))
 (segment (start 139.75 116.0723) (end 133.1777 109.5) (width 0.25) (layer "F.Cu") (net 12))
 (segment (start 133.1777 109.5) (end 132.825 109.5) (width 0.25) (layer "F.Cu") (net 12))
 (segment (start 139.75 123.25) (end 139.75 116.0723) (width 0.25) (layer "F.Cu") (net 12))
 (segment (start 142.25 129.25) (end 145.1318 129.25) (width 0.25) (layer "F.Cu") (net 5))
 (segment (start 158.09 113.03) (end 145.1562 113.03) (width 0.25) (layer "F.Cu") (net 5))
 (segment (start 145.1318 129.25) (end 145.1562 129.2256) (width 0.25) (layer "F.Cu") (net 5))
 (via (at 145.1562 129.2256) (size 0.6) (drill 0.3) (layers "F.Cu" "B.Cu") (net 5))
 (via (at 145.1562 113.03) (size 0.6) (drill 0.3) (layers "F.Cu" "B.Cu") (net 5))
 (segment (start 145.1562 113.03) (end 145.1562 129.2256) (width 0.25) (layer "B.Cu") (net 5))
 (segment (start 159.37 113.03) (end 159.37 114.4817) (width 0.25) (layer "F.Cu") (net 6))
 (segment (start 141.482 130.25) (end 140.9438 129.7118) (width 0.25) (layer "F.Cu") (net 6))
 (segment (start 142.25 130.25) (end 141.482 130.25) (width 0.25) (layer "F.Cu") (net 6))
 (segment (start 159.37 114.4817) (end 140.6096 114.4817) (width 0.25) (layer "F.Cu") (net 6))
 (segment (start 140.9438 129.7118) (end 140.6096 129.7118) (width 0.25) (layer "F.Cu") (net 6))
 (via (at 140.6096 129.7118) (size 0.6) (drill 0.3) (layers "F.Cu" "B.Cu") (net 6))
 (via (at 140.6096 114.4817) (size 0.6) (drill 0.3) (layers "F.Cu" "B.Cu") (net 6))
 (segment (start 140.6096 114.4817) (end 140.6096 129.7118) (width 0.25) (layer "B.Cu") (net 6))
 (segment (start 144.4745 128.75) (end 145.7363 127.4882) (width 0.25) (layer "F.Cu") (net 7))
 (segment (start 161.9 104.5183) (end 161.2646 103.8829) (width 0.25) (layer "F.Cu") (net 7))
 (segment (start 142.25 128.75) (end 144.4745 128.75) (width 0.25) (layer "F.Cu") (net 7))
 (segment (start 161.2646 103.8829) (end 146.0946 103.8829) (width 0.25) (layer "F.Cu") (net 7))
 (segment (start 145.7363 127.4882) (end 146.0946 127.4882) (width 0.25) (layer "F.Cu") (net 7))
 (segment (start 161.9 105.97) (end 161.9 104.5183) (width 0.25) (layer "F.Cu") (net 7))
 (via (at 146.0946 103.8829) (size 0.6) (drill 0.3) (layers "F.Cu" "B.Cu") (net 7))
 (via (at 146.0946 127.4882) (size 0.6) (drill 0.3) (layers "F.Cu" "B.Cu") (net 7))
 (segment (start 146.0946 103.8829) (end 146.0946 127.4882) (width 0.25) (layer "B.Cu") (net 7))
 (segment (start 160.63 104.5183) (end 154.0066 104.5183) (width 0.25) (layer "F.Cu") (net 8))
 (segment (start 160.63 105.97) (end 160.63 104.5183) (width 0.25) (layer "F.Cu") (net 8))
 (segment (start 149.5194 129.8567) (end 144.7232 129.8567) (width 0.25) (layer "F.Cu") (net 8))
 (segment (start 144.7232 129.8567) (end 144.6165 129.75) (width 0.25) (layer "F.Cu") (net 8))
 (segment (start 144.6165 129.75) (end 142.25 129.75) (width 0.25) (layer "F.Cu") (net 8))
 (via (at 154.0066 104.5183) (size 0.6) (drill 0.3) (layers "F.Cu" "B.Cu") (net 8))
 (via (at 149.5194 129.8567) (size 0.6) (drill 0.3) (layers "F.Cu" "B.Cu") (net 8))
 (segment (start 154.0066 125.3695) (end 154.0066 104.5183) (width 0.25) (layer "B.Cu") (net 8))
 (segment (start 149.5194 129.8567) (end 154.0066 125.3695) (width 0.25) (layer "B.Cu") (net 8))
 (segment (start 149.225 121.5) (end 142.501 121.5) (width 0.25) (layer "F.Cu") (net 4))
 (segment (start 140.75 131.75) (end 142.501 131.75) (width 0.25) (layer "F.Cu") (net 4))
 (via (at 142.501 131.75) (size 0.6) (drill 0.3) (layers "F.Cu" "B.Cu") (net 4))
 (via (at 142.501 121.5) (size 0.6) (drill 0.3) (layers "F.Cu" "B.Cu") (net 4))
 (segment (start 142.501 121.5) (end 142.501 131.75) (width 0.25) (layer "B.Cu") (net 4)))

